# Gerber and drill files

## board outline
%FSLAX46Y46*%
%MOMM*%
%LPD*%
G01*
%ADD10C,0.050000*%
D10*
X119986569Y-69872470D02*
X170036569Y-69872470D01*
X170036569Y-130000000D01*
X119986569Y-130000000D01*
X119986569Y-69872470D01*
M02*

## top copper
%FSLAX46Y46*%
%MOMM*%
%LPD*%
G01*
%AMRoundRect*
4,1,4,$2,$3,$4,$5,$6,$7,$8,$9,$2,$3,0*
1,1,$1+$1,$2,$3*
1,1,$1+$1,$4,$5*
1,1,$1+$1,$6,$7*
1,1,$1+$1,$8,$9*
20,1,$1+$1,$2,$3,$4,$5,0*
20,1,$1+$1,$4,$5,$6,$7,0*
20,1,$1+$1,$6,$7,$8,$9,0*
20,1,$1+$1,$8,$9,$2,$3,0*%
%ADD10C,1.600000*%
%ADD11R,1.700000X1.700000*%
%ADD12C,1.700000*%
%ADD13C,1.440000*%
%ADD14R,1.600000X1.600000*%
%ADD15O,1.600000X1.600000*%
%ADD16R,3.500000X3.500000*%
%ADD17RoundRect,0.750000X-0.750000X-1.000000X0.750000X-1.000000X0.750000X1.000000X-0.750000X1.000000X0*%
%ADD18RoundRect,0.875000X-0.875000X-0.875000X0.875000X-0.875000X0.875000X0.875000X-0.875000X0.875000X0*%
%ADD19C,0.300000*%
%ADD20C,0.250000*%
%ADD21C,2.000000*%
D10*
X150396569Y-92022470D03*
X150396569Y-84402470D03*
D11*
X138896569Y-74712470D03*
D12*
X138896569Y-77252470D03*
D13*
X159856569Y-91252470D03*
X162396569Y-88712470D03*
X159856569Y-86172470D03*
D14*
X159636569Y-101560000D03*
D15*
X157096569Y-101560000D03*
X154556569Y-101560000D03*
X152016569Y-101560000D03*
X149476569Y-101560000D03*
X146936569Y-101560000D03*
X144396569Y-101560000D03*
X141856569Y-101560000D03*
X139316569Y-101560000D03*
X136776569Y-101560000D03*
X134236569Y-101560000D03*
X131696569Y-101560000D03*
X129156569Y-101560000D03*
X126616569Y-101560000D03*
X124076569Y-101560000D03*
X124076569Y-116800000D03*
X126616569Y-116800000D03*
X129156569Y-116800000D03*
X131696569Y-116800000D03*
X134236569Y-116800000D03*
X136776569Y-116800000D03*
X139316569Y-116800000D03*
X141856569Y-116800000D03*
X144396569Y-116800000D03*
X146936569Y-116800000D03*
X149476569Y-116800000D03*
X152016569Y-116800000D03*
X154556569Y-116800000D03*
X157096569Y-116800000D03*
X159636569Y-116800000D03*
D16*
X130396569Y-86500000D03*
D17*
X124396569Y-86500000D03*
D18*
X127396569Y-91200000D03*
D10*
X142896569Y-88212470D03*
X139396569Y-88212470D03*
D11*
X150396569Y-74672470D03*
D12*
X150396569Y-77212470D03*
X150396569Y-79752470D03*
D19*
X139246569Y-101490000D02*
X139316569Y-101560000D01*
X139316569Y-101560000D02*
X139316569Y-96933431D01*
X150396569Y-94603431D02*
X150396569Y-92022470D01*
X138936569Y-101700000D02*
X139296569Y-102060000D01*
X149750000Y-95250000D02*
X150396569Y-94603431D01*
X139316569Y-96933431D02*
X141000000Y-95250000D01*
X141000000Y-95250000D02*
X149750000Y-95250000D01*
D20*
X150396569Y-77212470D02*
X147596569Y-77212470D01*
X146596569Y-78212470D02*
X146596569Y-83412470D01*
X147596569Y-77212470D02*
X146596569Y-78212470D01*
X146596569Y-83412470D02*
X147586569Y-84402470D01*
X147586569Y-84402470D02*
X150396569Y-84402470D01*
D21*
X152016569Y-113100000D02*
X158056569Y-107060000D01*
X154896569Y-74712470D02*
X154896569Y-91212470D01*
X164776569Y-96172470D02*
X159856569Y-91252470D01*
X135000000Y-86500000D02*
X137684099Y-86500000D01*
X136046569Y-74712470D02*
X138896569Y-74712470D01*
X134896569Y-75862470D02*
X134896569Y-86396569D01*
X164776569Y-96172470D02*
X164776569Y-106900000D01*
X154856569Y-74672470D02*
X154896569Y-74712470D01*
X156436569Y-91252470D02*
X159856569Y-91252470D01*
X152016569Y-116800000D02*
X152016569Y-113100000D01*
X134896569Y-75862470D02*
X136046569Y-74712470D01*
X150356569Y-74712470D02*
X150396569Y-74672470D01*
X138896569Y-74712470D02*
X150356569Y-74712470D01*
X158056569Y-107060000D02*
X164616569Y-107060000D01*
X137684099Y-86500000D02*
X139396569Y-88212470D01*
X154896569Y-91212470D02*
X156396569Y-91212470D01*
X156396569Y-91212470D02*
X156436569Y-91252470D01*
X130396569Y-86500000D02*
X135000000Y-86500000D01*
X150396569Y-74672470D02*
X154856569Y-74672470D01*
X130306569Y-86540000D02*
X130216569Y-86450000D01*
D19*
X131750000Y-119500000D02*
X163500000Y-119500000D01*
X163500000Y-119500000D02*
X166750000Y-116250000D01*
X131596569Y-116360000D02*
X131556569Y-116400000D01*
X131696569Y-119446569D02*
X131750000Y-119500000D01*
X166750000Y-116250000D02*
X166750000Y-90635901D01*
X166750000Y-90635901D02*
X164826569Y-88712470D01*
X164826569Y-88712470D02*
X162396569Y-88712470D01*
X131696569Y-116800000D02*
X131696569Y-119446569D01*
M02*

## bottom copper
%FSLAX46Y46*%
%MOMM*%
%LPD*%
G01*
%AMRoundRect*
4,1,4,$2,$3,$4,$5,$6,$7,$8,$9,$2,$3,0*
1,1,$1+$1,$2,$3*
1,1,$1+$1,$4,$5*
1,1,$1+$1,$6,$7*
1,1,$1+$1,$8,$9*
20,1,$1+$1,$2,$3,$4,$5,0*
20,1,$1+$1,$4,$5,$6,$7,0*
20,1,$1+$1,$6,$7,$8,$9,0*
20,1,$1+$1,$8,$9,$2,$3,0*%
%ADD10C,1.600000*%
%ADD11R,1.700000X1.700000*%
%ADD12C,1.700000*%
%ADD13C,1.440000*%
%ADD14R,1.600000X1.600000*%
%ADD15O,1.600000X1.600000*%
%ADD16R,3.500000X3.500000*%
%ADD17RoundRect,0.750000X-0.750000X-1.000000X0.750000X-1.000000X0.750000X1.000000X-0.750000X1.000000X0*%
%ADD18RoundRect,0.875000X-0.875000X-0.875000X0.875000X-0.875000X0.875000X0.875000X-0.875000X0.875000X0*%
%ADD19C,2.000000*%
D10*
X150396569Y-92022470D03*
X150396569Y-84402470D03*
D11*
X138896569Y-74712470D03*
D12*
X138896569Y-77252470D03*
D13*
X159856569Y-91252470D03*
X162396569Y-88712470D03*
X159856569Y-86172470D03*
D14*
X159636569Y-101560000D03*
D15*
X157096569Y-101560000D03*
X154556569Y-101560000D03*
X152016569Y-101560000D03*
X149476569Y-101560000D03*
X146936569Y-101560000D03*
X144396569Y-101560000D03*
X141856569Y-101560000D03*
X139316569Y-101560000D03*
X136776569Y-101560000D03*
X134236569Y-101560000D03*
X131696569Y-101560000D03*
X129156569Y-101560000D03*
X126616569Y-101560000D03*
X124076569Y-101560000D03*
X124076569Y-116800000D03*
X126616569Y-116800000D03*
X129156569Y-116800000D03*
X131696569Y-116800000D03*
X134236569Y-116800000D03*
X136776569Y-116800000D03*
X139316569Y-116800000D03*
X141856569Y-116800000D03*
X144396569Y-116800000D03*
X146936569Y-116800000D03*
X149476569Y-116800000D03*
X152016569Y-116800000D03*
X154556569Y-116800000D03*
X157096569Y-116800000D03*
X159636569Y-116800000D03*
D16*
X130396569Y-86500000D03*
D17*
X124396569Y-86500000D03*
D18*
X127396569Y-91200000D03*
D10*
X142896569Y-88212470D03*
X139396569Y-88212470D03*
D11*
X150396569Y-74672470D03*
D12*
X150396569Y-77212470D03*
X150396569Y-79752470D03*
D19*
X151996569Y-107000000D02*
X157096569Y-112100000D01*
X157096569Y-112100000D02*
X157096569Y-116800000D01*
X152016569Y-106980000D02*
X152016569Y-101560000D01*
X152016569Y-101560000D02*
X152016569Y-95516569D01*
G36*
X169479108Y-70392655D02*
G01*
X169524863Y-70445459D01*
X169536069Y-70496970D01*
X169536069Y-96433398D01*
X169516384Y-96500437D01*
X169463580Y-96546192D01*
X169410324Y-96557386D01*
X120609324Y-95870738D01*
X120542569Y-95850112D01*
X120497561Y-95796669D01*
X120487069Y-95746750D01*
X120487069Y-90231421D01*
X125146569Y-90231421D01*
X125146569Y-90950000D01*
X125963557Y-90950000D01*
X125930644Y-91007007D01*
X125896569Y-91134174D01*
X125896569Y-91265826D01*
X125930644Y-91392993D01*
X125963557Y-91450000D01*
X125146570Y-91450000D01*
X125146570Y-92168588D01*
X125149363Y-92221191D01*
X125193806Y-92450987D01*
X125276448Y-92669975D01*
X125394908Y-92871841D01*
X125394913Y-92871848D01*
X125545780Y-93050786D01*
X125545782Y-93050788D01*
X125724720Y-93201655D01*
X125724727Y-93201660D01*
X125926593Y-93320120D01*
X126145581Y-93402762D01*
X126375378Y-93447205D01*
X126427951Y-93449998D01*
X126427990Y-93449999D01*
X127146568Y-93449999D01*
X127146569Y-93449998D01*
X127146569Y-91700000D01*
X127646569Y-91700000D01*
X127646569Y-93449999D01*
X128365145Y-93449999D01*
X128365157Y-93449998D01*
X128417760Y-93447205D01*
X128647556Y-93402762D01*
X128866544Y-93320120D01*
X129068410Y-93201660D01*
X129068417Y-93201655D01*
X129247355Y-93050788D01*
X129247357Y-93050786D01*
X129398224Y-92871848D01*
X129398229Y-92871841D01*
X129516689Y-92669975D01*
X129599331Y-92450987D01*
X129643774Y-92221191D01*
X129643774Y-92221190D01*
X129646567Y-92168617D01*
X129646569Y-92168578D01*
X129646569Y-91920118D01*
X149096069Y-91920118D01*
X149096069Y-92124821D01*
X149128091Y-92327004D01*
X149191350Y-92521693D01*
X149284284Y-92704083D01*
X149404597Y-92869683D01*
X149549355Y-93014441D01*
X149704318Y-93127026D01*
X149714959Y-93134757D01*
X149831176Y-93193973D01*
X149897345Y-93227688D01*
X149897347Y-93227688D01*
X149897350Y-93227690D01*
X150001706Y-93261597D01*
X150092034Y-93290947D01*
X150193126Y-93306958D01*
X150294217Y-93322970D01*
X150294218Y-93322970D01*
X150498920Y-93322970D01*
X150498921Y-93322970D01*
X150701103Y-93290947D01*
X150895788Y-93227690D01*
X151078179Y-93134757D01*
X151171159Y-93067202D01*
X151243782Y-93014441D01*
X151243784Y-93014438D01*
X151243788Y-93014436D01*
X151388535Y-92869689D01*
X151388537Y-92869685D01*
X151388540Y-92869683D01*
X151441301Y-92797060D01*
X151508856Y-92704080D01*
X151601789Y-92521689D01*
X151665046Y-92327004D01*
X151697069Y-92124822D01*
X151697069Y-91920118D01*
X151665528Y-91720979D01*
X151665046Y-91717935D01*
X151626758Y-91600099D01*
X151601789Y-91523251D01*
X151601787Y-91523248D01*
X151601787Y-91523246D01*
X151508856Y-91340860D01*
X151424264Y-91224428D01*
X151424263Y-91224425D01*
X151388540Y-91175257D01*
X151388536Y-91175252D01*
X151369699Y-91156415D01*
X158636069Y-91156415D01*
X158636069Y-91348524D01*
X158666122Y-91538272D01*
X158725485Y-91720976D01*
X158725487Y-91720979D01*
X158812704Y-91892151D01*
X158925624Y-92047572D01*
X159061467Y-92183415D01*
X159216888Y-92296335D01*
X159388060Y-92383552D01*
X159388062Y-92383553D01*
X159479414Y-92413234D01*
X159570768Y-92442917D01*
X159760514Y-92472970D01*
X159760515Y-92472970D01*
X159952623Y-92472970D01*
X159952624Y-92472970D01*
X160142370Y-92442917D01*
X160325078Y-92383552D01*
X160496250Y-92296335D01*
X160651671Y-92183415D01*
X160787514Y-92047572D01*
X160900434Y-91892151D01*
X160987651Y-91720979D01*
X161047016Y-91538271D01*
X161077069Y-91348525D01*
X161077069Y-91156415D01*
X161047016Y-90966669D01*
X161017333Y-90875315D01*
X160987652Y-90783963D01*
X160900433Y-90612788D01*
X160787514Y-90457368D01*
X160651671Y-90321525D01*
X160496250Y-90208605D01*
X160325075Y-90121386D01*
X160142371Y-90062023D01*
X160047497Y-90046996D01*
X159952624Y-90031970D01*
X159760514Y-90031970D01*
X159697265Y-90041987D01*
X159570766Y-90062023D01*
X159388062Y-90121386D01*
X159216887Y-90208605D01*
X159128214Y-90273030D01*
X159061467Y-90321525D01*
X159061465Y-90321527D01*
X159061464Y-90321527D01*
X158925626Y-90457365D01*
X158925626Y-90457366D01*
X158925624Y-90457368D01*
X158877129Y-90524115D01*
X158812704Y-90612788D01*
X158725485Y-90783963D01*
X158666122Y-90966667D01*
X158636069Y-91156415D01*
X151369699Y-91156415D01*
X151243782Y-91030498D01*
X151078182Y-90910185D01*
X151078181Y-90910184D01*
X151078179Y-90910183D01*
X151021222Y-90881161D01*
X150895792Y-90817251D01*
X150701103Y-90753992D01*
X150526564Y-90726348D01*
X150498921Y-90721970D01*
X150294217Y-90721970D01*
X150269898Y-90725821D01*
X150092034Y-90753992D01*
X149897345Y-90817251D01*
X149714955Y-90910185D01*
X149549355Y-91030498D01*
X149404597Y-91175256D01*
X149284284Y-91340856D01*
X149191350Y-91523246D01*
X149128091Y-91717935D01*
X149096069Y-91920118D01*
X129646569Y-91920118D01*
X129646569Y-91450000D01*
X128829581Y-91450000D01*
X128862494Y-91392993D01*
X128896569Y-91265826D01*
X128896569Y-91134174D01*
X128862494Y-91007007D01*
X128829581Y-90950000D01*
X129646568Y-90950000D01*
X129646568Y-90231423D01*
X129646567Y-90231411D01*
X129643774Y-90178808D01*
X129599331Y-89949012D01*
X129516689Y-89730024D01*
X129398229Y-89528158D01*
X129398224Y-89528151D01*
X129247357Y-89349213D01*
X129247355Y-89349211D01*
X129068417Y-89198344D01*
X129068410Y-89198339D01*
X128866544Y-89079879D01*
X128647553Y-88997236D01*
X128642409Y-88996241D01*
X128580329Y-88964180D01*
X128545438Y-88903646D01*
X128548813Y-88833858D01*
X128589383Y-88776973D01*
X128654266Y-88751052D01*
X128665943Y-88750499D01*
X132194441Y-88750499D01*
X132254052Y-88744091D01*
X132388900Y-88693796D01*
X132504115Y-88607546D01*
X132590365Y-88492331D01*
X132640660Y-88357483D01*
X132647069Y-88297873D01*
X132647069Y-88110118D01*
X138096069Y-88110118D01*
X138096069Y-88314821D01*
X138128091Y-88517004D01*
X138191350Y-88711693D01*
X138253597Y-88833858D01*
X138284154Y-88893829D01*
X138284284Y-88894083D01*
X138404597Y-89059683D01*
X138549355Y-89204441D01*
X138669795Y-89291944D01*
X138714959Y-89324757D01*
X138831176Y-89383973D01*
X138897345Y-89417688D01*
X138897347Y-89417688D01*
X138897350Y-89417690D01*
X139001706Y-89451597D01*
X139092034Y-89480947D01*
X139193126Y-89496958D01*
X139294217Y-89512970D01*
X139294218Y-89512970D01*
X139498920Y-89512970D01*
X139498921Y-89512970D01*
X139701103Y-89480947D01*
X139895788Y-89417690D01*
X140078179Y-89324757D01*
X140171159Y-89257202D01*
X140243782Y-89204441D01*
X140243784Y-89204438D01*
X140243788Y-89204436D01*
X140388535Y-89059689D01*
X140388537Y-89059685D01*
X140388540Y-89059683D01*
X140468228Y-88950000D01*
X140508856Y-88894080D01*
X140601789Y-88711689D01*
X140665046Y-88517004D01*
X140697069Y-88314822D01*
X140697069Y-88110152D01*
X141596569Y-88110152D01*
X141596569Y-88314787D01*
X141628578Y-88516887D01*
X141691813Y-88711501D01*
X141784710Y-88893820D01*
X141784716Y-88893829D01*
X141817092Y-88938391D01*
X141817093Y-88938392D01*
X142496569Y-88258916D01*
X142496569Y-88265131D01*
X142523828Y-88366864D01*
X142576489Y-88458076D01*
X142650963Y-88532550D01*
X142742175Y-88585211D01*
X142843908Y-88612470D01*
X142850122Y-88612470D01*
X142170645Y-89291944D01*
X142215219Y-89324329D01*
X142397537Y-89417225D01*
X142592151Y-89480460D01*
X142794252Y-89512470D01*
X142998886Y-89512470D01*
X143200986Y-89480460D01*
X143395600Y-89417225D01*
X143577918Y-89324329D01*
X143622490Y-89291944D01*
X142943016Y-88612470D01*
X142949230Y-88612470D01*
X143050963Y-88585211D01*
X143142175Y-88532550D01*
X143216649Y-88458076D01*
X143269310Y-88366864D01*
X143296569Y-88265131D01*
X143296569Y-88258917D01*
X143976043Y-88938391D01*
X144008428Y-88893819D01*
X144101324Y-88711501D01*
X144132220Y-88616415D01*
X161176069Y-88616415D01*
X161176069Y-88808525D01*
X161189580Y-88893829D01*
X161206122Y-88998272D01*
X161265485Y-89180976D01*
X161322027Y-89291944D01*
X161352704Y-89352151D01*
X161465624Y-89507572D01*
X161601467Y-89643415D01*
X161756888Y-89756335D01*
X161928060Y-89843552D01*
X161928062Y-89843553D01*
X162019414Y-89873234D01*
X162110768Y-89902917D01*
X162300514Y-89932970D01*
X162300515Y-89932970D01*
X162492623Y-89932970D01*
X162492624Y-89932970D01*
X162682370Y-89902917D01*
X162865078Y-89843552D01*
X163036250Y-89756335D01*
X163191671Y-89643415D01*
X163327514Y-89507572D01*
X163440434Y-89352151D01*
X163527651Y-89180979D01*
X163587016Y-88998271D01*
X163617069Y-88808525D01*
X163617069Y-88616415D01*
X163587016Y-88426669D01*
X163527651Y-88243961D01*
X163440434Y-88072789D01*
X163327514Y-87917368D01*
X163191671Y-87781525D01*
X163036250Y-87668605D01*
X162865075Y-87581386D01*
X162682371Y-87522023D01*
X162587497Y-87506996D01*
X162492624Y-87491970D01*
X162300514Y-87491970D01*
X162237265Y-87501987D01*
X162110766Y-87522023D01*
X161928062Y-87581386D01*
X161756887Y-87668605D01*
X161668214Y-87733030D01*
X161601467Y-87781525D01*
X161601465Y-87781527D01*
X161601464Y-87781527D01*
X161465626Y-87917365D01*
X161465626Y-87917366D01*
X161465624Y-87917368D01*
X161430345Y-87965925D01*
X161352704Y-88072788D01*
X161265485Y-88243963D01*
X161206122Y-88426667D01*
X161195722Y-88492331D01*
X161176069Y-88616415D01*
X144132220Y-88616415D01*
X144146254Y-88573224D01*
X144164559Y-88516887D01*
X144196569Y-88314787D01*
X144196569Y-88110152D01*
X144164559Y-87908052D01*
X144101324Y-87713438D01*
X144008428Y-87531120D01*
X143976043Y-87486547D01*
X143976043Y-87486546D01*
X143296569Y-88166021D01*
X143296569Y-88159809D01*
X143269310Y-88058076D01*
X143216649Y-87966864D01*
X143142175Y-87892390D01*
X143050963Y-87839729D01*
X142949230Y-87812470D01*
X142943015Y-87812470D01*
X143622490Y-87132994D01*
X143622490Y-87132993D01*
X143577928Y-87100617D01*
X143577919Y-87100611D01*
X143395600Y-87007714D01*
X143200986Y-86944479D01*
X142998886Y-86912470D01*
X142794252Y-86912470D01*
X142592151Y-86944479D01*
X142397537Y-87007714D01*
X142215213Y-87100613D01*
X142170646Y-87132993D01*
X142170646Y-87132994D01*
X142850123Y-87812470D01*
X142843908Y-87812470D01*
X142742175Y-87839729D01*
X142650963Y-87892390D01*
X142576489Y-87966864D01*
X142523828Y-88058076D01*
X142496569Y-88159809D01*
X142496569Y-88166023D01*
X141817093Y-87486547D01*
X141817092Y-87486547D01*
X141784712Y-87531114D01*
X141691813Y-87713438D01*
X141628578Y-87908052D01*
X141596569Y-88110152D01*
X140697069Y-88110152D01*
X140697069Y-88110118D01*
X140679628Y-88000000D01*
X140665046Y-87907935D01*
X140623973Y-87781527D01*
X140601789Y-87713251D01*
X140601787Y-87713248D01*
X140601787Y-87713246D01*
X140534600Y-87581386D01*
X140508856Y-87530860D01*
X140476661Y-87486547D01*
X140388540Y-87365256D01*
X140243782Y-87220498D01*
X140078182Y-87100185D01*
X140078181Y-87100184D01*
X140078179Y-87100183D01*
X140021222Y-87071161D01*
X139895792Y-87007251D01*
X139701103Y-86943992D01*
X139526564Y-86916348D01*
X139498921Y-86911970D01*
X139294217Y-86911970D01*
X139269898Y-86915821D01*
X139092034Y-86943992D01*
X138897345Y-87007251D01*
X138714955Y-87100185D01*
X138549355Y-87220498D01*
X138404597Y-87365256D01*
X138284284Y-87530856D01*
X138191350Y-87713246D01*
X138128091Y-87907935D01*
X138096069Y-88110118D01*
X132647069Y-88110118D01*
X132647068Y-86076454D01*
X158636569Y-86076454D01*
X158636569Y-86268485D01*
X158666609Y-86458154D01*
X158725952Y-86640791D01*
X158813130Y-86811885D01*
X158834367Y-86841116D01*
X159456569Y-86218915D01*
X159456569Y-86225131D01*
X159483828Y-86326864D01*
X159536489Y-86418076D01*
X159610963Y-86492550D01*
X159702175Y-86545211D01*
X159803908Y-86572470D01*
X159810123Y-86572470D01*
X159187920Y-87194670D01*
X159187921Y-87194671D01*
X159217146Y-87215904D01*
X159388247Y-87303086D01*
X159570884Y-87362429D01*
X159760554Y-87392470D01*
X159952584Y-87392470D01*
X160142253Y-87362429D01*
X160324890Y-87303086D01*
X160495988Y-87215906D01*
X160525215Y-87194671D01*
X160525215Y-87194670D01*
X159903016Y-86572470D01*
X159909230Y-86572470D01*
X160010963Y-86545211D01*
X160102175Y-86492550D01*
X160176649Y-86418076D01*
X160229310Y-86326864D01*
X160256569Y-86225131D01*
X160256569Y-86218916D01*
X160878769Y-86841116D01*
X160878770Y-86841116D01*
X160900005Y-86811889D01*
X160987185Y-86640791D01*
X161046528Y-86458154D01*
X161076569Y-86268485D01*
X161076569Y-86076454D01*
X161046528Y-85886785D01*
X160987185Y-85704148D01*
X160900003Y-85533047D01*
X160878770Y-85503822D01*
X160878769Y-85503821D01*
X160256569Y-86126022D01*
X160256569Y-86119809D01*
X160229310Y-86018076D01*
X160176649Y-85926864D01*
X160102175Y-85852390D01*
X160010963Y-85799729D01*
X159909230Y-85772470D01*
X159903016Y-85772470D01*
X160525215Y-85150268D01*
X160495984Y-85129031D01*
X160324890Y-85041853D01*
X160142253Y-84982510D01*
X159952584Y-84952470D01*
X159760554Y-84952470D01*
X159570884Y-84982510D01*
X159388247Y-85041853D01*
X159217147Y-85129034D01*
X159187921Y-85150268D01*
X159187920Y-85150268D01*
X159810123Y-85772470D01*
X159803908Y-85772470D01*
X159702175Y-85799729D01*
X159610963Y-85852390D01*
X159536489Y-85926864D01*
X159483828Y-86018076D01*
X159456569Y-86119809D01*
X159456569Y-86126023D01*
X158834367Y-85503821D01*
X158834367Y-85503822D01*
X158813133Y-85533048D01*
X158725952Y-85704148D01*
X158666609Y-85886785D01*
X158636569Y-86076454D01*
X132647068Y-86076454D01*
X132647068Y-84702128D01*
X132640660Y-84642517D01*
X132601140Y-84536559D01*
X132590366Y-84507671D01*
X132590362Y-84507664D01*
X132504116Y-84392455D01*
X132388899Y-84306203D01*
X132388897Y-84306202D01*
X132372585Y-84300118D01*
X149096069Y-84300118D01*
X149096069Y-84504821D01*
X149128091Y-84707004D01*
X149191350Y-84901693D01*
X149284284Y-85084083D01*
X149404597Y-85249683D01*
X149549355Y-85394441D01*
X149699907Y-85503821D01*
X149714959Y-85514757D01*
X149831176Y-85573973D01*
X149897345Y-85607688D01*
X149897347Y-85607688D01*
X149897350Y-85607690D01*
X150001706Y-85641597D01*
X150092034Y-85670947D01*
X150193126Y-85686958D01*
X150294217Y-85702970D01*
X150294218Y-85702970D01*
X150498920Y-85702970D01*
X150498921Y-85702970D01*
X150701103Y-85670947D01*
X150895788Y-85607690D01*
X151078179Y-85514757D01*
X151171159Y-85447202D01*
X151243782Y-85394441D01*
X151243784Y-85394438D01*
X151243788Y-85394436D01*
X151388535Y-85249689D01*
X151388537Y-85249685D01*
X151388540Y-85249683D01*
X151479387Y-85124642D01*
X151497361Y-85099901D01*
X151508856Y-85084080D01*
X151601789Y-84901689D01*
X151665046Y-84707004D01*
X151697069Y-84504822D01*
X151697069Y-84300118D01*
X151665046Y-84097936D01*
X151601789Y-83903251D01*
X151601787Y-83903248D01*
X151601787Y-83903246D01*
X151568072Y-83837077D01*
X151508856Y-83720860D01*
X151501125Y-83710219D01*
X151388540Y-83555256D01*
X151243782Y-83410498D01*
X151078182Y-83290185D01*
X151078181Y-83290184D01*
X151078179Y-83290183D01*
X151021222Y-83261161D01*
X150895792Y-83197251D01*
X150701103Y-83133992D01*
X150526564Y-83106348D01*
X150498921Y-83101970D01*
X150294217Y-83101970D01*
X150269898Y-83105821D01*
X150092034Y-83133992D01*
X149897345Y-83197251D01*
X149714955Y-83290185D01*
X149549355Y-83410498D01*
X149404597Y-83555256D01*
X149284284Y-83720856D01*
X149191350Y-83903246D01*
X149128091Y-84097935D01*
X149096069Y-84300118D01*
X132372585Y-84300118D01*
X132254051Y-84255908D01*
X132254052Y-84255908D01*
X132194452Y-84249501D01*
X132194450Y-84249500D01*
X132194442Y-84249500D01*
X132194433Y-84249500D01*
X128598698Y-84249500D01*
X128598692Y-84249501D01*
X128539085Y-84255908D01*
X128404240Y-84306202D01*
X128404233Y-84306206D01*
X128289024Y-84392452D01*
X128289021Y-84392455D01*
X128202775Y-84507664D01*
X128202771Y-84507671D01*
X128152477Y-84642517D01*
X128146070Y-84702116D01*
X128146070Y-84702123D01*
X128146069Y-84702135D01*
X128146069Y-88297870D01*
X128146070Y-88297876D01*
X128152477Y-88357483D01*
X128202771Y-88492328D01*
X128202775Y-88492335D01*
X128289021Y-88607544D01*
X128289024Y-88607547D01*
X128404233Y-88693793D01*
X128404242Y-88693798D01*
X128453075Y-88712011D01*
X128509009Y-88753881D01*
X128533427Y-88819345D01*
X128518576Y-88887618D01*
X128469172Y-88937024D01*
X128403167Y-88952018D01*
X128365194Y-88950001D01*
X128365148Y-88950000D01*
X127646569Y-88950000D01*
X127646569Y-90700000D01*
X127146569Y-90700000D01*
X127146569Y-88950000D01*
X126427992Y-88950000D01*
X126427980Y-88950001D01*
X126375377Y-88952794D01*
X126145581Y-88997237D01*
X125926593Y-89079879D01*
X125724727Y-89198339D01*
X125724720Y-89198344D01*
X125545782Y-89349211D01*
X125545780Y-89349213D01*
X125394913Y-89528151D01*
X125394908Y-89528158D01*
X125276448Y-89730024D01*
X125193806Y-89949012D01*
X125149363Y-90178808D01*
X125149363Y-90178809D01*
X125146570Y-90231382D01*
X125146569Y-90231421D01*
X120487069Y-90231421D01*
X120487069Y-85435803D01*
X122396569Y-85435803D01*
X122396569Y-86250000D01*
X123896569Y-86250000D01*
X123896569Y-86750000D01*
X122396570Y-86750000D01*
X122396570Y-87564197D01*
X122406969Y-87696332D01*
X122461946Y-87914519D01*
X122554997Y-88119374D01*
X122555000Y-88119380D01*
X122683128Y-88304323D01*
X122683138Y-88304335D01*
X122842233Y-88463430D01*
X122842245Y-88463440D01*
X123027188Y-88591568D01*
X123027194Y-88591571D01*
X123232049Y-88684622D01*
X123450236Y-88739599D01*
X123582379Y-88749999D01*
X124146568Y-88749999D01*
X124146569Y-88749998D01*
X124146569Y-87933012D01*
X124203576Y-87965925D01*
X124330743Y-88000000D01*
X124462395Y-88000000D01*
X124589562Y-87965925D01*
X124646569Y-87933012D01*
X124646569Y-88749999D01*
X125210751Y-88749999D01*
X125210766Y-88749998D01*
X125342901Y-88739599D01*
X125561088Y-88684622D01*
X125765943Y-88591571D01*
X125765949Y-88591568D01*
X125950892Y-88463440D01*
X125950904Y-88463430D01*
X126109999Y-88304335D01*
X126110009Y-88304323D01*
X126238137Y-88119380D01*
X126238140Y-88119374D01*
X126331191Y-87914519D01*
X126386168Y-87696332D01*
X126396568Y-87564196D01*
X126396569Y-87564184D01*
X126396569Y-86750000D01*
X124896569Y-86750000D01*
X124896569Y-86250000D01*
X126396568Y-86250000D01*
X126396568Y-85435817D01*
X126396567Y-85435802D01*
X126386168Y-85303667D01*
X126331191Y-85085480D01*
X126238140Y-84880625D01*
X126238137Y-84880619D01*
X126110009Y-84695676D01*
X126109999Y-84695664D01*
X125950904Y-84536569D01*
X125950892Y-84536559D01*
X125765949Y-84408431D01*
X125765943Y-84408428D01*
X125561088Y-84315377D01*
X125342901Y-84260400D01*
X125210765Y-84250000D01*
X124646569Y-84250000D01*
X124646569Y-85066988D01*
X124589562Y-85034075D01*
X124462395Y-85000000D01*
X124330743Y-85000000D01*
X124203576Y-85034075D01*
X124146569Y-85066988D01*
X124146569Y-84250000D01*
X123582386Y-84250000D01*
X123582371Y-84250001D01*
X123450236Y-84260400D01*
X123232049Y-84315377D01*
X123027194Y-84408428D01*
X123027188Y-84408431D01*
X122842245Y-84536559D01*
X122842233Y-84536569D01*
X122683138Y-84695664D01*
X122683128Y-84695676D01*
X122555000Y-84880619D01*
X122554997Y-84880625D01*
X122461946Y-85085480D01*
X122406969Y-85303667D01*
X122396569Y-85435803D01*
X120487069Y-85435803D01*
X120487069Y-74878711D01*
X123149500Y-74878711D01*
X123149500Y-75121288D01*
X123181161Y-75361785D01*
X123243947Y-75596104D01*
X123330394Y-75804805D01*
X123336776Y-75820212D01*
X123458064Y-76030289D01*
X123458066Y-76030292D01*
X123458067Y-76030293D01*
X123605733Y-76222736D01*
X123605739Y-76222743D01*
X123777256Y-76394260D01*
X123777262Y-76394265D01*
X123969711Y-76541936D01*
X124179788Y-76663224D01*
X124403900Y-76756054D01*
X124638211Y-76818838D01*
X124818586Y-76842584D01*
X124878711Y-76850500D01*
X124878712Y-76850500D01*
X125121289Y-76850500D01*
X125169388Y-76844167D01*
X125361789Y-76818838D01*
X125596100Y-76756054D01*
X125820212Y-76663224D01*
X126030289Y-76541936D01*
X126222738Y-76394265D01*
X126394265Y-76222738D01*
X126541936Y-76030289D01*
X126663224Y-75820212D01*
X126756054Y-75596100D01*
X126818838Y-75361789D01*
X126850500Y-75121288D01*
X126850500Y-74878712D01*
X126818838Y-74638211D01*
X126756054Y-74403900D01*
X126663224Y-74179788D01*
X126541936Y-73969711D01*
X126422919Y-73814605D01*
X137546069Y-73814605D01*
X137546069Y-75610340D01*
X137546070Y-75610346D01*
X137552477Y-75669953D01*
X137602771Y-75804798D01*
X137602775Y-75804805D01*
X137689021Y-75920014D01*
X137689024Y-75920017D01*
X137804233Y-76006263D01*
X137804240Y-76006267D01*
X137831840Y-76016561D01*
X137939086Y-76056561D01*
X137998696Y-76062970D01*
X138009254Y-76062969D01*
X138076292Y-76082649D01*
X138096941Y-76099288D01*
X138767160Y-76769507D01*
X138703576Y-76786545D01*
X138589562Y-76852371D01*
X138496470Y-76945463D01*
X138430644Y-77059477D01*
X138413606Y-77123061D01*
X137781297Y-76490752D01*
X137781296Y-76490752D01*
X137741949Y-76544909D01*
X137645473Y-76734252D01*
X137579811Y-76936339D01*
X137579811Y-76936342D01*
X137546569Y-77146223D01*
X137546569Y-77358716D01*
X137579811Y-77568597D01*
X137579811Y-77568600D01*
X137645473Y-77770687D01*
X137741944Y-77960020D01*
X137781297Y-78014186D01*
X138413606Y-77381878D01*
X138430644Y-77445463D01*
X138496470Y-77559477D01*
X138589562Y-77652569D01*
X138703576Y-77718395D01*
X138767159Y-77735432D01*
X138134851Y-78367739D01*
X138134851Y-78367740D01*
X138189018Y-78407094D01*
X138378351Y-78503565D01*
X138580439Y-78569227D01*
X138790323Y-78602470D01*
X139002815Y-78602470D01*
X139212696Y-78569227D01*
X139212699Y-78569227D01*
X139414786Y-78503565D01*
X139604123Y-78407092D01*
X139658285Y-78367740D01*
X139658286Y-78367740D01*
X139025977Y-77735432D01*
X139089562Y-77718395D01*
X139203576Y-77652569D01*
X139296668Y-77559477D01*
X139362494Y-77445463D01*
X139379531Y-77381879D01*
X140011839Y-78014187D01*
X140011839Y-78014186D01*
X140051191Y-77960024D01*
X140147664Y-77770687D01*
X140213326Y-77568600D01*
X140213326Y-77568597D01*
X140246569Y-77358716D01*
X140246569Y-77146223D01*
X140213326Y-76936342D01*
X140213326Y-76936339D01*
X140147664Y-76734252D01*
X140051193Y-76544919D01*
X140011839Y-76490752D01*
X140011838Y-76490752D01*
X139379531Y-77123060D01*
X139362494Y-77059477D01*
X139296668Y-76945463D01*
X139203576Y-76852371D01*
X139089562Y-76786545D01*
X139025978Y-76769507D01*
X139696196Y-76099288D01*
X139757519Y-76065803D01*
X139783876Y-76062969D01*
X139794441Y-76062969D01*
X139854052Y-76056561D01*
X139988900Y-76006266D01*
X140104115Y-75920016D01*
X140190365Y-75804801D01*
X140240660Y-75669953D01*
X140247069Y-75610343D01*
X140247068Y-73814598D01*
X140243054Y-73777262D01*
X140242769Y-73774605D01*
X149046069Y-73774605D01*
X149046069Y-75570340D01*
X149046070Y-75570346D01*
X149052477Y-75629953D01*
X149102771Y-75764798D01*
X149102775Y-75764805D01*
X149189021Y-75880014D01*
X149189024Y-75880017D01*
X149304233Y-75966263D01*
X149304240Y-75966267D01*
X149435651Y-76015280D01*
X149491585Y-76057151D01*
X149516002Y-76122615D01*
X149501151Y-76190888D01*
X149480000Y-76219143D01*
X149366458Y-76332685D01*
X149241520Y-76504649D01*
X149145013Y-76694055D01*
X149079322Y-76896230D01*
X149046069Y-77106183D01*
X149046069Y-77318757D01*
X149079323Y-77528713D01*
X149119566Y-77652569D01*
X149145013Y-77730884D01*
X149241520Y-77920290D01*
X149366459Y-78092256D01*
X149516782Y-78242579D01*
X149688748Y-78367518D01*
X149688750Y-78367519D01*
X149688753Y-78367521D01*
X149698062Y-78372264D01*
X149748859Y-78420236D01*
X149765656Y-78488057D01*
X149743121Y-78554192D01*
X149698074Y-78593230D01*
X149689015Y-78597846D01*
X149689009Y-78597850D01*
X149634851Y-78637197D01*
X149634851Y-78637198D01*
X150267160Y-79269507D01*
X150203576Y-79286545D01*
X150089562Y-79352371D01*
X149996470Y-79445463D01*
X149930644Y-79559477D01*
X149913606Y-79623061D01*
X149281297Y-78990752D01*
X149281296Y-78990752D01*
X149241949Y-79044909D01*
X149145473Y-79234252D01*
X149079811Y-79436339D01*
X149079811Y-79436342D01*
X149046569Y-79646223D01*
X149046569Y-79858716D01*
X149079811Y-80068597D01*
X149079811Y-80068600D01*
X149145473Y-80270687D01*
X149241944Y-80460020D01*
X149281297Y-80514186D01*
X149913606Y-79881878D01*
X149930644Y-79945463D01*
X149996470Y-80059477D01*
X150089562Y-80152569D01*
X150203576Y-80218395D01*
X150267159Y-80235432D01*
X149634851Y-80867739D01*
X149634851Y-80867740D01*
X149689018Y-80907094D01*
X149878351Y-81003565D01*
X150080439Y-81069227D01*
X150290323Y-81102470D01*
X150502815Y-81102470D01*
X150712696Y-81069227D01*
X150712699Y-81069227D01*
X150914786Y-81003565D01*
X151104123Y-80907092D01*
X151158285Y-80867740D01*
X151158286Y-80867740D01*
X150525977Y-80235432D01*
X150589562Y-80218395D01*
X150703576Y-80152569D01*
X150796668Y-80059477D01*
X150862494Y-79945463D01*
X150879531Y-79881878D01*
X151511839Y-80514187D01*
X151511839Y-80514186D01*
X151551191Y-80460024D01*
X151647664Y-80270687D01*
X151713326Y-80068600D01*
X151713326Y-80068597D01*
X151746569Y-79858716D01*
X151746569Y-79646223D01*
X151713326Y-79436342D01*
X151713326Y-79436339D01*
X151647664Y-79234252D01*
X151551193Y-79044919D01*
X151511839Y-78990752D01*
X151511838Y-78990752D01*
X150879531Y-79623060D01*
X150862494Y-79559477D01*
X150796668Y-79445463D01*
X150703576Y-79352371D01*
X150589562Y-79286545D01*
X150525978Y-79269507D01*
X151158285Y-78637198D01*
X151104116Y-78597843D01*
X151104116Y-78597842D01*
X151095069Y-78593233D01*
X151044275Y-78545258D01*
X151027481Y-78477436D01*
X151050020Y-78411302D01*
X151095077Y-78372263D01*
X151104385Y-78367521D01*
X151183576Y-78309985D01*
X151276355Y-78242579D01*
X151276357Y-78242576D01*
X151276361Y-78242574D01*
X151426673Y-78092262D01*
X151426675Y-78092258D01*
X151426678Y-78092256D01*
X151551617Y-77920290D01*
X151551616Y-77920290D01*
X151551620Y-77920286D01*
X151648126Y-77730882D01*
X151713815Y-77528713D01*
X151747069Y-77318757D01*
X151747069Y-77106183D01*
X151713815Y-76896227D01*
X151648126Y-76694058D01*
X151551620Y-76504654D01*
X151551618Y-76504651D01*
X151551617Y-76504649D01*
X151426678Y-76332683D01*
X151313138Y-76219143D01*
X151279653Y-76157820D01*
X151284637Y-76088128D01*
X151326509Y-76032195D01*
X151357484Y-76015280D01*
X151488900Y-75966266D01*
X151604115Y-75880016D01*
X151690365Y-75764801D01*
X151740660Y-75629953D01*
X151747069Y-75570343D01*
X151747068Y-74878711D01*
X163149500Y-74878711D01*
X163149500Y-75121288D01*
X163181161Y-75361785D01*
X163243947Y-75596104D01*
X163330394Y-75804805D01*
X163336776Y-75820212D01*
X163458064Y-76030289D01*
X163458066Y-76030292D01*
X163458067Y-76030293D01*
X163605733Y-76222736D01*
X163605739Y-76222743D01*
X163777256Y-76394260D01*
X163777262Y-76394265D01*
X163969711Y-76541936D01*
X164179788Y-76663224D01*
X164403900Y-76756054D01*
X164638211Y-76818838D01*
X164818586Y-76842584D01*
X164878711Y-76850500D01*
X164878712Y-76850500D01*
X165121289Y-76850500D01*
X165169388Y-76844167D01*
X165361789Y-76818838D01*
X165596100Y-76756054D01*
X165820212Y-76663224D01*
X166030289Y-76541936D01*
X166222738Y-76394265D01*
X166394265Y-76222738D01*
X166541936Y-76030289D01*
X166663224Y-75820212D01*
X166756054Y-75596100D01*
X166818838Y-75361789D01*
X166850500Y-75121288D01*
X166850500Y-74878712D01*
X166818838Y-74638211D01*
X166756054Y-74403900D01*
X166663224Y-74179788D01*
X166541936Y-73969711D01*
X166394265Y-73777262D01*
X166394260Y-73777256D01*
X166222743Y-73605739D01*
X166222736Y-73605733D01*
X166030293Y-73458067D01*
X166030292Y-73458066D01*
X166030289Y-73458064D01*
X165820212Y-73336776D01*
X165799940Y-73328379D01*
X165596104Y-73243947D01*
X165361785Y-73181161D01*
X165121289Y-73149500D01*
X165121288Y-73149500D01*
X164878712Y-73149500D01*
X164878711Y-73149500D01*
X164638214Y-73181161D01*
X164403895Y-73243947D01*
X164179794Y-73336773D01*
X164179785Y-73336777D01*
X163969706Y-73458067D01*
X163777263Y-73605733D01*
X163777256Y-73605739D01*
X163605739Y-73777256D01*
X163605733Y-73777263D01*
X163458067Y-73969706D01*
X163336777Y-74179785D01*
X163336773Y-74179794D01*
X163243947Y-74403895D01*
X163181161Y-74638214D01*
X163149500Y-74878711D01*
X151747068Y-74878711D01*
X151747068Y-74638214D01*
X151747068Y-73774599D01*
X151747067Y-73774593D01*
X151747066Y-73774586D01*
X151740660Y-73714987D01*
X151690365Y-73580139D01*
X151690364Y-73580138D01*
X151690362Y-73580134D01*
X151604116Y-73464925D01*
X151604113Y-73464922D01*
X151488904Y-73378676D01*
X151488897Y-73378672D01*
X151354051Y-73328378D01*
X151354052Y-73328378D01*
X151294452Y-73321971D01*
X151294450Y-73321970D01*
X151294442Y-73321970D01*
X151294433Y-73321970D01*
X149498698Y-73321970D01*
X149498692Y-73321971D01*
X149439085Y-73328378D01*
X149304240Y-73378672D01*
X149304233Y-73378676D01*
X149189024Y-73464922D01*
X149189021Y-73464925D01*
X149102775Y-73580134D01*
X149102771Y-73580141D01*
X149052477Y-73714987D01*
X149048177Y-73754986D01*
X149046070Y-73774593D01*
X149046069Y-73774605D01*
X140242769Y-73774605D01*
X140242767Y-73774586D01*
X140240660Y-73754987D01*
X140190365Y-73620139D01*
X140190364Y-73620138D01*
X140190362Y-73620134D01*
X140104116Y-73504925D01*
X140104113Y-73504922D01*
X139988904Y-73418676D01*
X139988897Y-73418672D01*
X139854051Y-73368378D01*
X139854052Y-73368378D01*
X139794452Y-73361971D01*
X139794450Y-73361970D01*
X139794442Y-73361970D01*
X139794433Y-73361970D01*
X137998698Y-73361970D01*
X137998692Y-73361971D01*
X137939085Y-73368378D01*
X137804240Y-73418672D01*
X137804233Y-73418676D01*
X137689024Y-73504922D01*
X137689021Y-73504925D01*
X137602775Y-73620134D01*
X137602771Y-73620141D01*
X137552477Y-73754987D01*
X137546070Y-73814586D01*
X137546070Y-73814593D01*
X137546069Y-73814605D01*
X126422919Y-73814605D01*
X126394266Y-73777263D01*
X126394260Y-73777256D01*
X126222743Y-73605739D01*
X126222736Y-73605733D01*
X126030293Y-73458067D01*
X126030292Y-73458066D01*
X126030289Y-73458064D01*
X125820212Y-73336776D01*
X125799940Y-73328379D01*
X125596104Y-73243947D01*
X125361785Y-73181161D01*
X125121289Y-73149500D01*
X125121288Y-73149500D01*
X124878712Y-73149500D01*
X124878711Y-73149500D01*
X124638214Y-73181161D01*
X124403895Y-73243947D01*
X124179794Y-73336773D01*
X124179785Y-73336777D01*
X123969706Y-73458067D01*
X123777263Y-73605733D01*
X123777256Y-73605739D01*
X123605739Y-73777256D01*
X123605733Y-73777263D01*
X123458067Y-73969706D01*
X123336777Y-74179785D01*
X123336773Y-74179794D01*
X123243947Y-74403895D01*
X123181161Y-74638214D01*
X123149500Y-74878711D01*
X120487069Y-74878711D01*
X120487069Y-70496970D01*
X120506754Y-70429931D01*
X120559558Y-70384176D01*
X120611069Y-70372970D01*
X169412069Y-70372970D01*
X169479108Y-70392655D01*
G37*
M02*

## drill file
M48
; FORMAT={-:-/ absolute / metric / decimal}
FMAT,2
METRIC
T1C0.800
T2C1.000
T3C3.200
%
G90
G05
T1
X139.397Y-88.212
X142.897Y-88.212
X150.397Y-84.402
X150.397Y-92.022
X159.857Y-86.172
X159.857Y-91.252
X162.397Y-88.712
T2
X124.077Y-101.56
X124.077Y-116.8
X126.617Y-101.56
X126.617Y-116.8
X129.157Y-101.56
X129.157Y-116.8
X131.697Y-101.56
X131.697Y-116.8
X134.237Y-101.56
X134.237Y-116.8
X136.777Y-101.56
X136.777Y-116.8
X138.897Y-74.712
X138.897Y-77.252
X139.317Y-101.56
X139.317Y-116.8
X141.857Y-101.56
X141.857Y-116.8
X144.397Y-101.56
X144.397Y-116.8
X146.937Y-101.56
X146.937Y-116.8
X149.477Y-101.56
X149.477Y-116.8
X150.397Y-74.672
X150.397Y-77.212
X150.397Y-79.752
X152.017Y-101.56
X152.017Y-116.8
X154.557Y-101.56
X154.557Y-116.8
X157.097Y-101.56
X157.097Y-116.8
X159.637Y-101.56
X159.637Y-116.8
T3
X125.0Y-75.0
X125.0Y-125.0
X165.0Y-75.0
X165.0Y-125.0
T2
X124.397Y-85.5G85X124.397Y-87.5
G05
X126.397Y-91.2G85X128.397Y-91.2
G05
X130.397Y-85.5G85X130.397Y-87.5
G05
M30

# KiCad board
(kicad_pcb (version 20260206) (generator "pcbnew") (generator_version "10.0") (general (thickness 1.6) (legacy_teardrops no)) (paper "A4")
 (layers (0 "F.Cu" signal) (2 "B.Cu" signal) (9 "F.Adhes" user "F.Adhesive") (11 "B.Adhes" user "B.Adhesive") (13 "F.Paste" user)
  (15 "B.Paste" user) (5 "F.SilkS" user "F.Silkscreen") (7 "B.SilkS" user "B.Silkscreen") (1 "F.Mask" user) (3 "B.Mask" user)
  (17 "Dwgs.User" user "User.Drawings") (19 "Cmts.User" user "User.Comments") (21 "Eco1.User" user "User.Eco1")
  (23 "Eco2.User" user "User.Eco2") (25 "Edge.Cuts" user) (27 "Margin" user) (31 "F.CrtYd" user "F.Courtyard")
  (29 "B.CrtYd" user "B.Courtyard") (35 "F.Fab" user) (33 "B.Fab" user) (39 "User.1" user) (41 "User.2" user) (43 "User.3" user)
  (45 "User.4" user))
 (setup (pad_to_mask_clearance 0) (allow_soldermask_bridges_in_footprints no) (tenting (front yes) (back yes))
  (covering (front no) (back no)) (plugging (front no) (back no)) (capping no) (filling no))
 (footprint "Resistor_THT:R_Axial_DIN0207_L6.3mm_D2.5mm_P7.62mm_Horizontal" (layer "F.Cu") (at 150.396569 92.02247 90)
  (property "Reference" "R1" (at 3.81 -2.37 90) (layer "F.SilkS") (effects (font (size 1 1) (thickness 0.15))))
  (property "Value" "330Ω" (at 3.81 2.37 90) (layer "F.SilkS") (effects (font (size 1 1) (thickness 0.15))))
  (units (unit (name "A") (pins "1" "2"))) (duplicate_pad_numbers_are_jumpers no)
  (pad "1" thru_hole circle (at 0 0 90) (size 1.6 1.6) (drill 0.8) (layers "*.Cu" "*.Mask") (remove_unused_layers no) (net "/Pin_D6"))
  (pad "2" thru_hole circle (at 7.62 0 90) (size 1.6 1.6) (drill 0.8) (layers "*.Cu" "*.Mask") (remove_unused_layers no) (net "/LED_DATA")))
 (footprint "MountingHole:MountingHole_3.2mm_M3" (layer "F.Cu") (at 165 125)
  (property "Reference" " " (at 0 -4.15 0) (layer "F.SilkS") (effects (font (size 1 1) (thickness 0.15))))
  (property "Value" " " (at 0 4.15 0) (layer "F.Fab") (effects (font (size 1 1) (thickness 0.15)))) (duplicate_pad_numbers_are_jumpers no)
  (pad "" np_thru_hole circle (at 0 0) (size 3.2 3.2) (drill 3.2) (layers "*.Cu" "*.Mask")))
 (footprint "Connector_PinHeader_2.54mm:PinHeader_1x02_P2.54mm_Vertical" (layer "F.Cu") (at 138.896569 74.71247)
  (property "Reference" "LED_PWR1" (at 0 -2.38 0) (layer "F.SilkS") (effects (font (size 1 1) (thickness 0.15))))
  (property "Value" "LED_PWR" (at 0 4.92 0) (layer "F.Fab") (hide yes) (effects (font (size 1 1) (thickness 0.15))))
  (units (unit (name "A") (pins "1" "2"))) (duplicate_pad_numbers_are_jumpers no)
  (pad "1" thru_hole rect (at 0 0) (size 1.7 1.7) (drill 1) (layers "*.Cu" "*.Mask") (remove_unused_layers no) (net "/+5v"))
  (pad "2" thru_hole circle (at 0 2.54) (size 1.7 1.7) (drill 1) (layers "*.Cu" "*.Mask") (remove_unused_layers no) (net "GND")))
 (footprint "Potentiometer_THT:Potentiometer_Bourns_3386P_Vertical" (layer "F.Cu") (at 159.856569 91.25247)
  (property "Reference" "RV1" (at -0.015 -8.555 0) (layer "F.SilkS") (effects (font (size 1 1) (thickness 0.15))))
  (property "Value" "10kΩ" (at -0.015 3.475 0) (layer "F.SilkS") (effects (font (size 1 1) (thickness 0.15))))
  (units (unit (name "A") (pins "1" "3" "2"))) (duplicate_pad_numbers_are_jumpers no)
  (pad "1" thru_hole circle (at 0 0) (size 1.44 1.44) (drill 0.8) (layers "*.Cu" "*.Mask") (remove_unused_layers no) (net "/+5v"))
  (pad "2" thru_hole circle (at 2.54 -2.54) (size 1.44 1.44) (drill 0.8) (layers "*.Cu" "*.Mask") (remove_unused_layers no)
   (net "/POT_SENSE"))
  (pad "3" thru_hole circle (at 0 -5.08) (size 1.44 1.44) (drill 0.8) (layers "*.Cu" "*.Mask") (remove_unused_layers no) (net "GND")))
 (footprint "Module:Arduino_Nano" (layer "F.Cu") (at 159.636569 101.56 -90)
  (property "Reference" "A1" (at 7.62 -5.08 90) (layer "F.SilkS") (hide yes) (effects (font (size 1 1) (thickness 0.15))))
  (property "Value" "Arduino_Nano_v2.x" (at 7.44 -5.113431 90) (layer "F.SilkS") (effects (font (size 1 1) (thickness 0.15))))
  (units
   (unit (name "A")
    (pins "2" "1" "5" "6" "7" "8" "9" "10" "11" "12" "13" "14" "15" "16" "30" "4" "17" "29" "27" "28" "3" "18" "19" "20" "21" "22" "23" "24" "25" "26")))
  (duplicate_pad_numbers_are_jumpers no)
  (pad "1" thru_hole rect (at 0 0 270) (size 1.6 1.6) (drill 1) (layers "*.Cu" "*.Mask") (remove_unused_layers no)
   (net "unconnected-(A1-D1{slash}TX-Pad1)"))
  (pad "2" thru_hole oval (at 0 2.54 270) (size 1.6 1.6) (drill 1) (layers "*.Cu" "*.Mask") (remove_unused_layers no)
   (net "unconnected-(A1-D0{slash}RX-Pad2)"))
  (pad "3" thru_hole oval (at 0 5.08 270) (size 1.6 1.6) (drill 1) (layers "*.Cu" "*.Mask") (remove_unused_layers no)
   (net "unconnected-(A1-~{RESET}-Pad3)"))
  (pad "4" thru_hole oval (at 0 7.62 270) (size 1.6 1.6) (drill 1) (layers "*.Cu" "*.Mask") (remove_unused_layers no) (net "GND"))
  (pad "5" thru_hole oval (at 0 10.16 270) (size 1.6 1.6) (drill 1) (layers "*.Cu" "*.Mask") (remove_unused_layers no)
   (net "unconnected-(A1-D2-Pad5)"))
  (pad "6" thru_hole oval (at 0 12.7 270) (size 1.6 1.6) (drill 1) (layers "*.Cu" "*.Mask") (remove_unused_layers no)
   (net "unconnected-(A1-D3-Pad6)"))
  (pad "7" thru_hole oval (at 0 15.24 270) (size 1.6 1.6) (drill 1) (layers "*.Cu" "*.Mask") (remove_unused_layers no)
   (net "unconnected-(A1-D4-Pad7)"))
  (pad "8" thru_hole oval (at 0 17.78 270) (size 1.6 1.6) (drill 1) (layers "*.Cu" "*.Mask") (remove_unused_layers no)
   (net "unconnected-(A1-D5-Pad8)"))
  (pad "9" thru_hole oval (at 0 20.32 270) (size 1.6 1.6) (drill 1) (layers "*.Cu" "*.Mask") (remove_unused_layers no) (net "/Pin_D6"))
  (pad "10" thru_hole oval (at 0 22.86 270) (size 1.6 1.6) (drill 1) (layers "*.Cu" "*.Mask") (remove_unused_layers no)
   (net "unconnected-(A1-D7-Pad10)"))
  (pad "11" thru_hole oval (at 0 25.4 270) (size 1.6 1.6) (drill 1) (layers "*.Cu" "*.Mask") (remove_unused_layers no)
   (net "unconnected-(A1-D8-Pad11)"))
  (pad "12" thru_hole oval (at 0 27.94 270) (size 1.6 1.6) (drill 1) (layers "*.Cu" "*.Mask") (remove_unused_layers no)
   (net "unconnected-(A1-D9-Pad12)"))
  (pad "13" thru_hole oval (at 0 30.48 270) (size 1.6 1.6) (drill 1) (layers "*.Cu" "*.Mask") (remove_unused_layers no)
   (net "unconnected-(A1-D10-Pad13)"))
  (pad "14" thru_hole oval (at 0 33.02 270) (size 1.6 1.6) (drill 1) (layers "*.Cu" "*.Mask") (remove_unused_layers no)
   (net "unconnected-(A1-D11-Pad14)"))
  (pad "15" thru_hole oval (at 0 35.56 270) (size 1.6 1.6) (drill 1) (layers "*.Cu" "*.Mask") (remove_unused_layers no)
   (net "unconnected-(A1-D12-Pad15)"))
  (pad "16" thru_hole oval (at 15.24 35.56 270) (size 1.6 1.6) (drill 1) (layers "*.Cu" "*.Mask") (remove_unused_layers no)
   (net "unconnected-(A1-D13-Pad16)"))
  (pad "17" thru_hole oval (at 15.24 33.02 270) (size 1.6 1.6) (drill 1) (layers "*.Cu" "*.Mask") (remove_unused_layers no)
   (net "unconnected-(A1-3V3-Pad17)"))
  (pad "18" thru_hole oval (at 15.24 30.48 270) (size 1.6 1.6) (drill 1) (layers "*.Cu" "*.Mask") (remove_unused_layers no)
   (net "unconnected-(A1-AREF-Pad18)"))
  (pad "19" thru_hole oval (at 15.24 27.94 270) (size 1.6 1.6) (drill 1) (layers "*.Cu" "*.Mask") (remove_unused_layers no)
   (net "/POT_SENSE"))
  (pad "20" thru_hole oval (at 15.24 25.4 270) (size 1.6 1.6) (drill 1) (layers "*.Cu" "*.Mask") (remove_unused_layers no)
   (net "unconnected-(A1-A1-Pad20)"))
  (pad "21" thru_hole oval (at 15.24 22.86 270) (size 1.6 1.6) (drill 1) (layers "*.Cu" "*.Mask") (remove_unused_layers no)
   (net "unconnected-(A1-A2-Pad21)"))
  (pad "22" thru_hole oval (at 15.24 20.32 270) (size 1.6 1.6) (drill 1) (layers "*.Cu" "*.Mask") (remove_unused_layers no)
   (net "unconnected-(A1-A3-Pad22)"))
  (pad "23" thru_hole oval (at 15.24 17.78 270) (size 1.6 1.6) (drill 1) (layers "*.Cu" "*.Mask") (remove_unused_layers no)
   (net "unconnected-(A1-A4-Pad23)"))
  (pad "24" thru_hole oval (at 15.24 15.24 270) (size 1.6 1.6) (drill 1) (layers "*.Cu" "*.Mask") (remove_unused_layers no)
   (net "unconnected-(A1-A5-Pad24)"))
  (pad "25" thru_hole oval (at 15.24 12.7 270) (size 1.6 1.6) (drill 1) (layers "*.Cu" "*.Mask") (remove_unused_layers no)
   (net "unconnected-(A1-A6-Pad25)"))
  (pad "26" thru_hole oval (at 15.24 10.16 270) (size 1.6 1.6) (drill 1) (layers "*.Cu" "*.Mask") (remove_unused_layers no)
   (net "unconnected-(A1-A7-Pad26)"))
  (pad "27" thru_hole oval (at 15.24 7.62 270) (size 1.6 1.6) (drill 1) (layers "*.Cu" "*.Mask") (remove_unused_layers no) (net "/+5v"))
  (pad "28" thru_hole oval (at 15.24 5.08 270) (size 1.6 1.6) (drill 1) (layers "*.Cu" "*.Mask") (remove_unused_layers no)
   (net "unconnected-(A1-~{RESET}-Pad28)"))
  (pad "29" thru_hole oval (at 15.24 2.54 270) (size 1.6 1.6) (drill 1) (layers "*.Cu" "*.Mask") (remove_unused_layers no) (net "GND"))
  (pad "30" thru_hole oval (at 15.24 0 270) (size 1.6 1.6) (drill 1) (layers "*.Cu" "*.Mask") (remove_unused_layers no)
   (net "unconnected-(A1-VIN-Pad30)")))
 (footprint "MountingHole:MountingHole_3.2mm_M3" (layer "F.Cu") (at 125 75)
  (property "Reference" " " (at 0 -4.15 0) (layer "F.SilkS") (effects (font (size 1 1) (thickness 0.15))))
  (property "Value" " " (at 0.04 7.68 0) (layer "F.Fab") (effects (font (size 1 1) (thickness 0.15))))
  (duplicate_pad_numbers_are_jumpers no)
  (pad "" np_thru_hole circle (at 0 0) (size 3.2 3.2) (drill 3.2) (layers "*.Cu" "*.Mask")))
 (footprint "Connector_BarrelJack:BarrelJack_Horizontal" (layer "F.Cu") (at 130.396569 86.5)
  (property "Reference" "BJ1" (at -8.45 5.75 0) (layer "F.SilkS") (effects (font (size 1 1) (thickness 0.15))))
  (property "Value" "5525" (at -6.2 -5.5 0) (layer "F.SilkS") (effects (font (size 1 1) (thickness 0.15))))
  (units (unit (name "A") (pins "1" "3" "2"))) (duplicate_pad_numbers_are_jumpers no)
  (pad "1" thru_hole rect (at 0 0) (size 3.5 3.5) (drill oval 1 3) (layers "*.Cu" "*.Mask") (remove_unused_layers no) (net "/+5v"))
  (pad "2" thru_hole roundrect (at -6 0) (size 3 3.5) (drill oval 1 3) (layers "*.Cu" "*.Mask") (remove_unused_layers no)
   (roundrect_rratio 0.25) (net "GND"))
  (pad "3" thru_hole roundrect (at -3 4.7) (size 3.5 3.5) (drill oval 3 1) (layers "*.Cu" "*.Mask") (remove_unused_layers no)
   (roundrect_rratio 0.25) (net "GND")))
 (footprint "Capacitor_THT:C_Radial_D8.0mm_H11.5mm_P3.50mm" (layer "F.Cu") (at 142.896569 88.21247 180)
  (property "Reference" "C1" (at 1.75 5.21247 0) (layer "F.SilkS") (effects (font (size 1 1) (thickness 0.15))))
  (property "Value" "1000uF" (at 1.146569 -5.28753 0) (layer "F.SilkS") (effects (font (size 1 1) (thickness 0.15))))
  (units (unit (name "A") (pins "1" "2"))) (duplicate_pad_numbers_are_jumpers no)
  (pad "1" thru_hole circle (at 0 0 180) (size 1.6 1.6) (drill 0.8) (layers "*.Cu" "*.Mask") (remove_unused_layers no) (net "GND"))
  (pad "2" thru_hole circle (at 3.5 0 180) (size 1.6 1.6) (drill 0.8) (layers "*.Cu" "*.Mask") (remove_unused_layers no) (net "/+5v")))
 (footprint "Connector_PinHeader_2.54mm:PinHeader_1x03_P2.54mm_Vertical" (layer "F.Cu") (at 150.396569 74.67247)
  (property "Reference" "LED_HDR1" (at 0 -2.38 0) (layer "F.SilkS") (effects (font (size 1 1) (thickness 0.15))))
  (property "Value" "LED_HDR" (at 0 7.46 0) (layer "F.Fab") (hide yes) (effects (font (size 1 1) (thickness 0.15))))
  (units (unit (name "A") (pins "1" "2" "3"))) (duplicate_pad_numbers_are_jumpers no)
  (pad "1" thru_hole rect (at 0 0) (size 1.7 1.7) (drill 1) (layers "*.Cu" "*.Mask") (remove_unused_layers no) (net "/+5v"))
  (pad "2" thru_hole circle (at 0 2.54) (size 1.7 1.7) (drill 1) (layers "*.Cu" "*.Mask") (remove_unused_layers no) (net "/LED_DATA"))
  (pad "3" thru_hole circle (at 0 5.08) (size 1.7 1.7) (drill 1) (layers "*.Cu" "*.Mask") (remove_unused_layers no) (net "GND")))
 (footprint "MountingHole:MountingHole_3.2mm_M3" (layer "F.Cu") (at 165 75)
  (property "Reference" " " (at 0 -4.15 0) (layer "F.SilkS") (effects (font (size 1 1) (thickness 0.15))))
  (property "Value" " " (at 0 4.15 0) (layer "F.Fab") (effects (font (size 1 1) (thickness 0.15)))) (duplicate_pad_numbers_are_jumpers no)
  (pad "" np_thru_hole circle (at 0 0) (size 3.2 3.2) (drill 3.2) (layers "*.Cu" "*.Mask")))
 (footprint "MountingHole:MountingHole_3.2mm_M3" (layer "F.Cu") (at 125 125)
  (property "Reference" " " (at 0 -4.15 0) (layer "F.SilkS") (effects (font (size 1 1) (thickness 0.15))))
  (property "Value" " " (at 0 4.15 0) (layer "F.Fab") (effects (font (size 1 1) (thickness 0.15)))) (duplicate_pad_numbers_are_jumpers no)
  (pad "" np_thru_hole circle (at 0 0) (size 3.2 3.2) (drill 3.2) (layers "*.Cu" "*.Mask")))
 (gr_rect (start 119.986569 69.87247) (end 170.036569 130) (stroke (width 0.05) (type default)) (fill no) (layer "Edge.Cuts"))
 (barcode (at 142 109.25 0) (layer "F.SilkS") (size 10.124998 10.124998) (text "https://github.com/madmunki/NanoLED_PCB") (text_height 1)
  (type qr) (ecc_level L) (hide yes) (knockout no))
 (segment (start 139.246569 101.49) (end 139.316569 101.56) (width 0.3) (layer "F.Cu") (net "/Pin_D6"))
 (segment (start 139.316569 101.56) (end 139.316569 96.933431) (width 0.3) (layer "F.Cu") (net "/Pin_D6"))
 (segment (start 150.396569 94.603431) (end 150.396569 92.02247) (width 0.3) (layer "F.Cu") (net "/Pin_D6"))
 (segment (start 138.936569 101.7) (end 139.296569 102.06) (width 0.3) (layer "F.Cu") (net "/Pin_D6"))
 (segment (start 149.75 95.25) (end 150.396569 94.603431) (width 0.3) (layer "F.Cu") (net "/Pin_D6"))
 (segment (start 139.316569 96.933431) (end 141 95.25) (width 0.3) (layer "F.Cu") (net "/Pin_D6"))
 (segment (start 141 95.25) (end 149.75 95.25) (width 0.3) (layer "F.Cu") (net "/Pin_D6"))
 (segment (start 150.396569 77.21247) (end 147.596569 77.21247) (width 0.25) (layer "F.Cu") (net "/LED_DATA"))
 (segment (start 146.596569 78.21247) (end 146.596569 83.41247) (width 0.25) (layer "F.Cu") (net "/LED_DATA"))
 (segment (start 147.596569 77.21247) (end 146.596569 78.21247) (width 0.25) (layer "F.Cu") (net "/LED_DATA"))
 (segment (start 146.596569 83.41247) (end 147.586569 84.40247) (width 0.25) (layer "F.Cu") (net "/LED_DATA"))
 (segment (start 147.586569 84.40247) (end 150.396569 84.40247) (width 0.25) (layer "F.Cu") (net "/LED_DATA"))
 (segment (start 152.016569 113.1) (end 158.056569 107.06) (width 2) (layer "F.Cu") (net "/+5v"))
 (segment (start 154.896569 74.71247) (end 154.896569 91.21247) (width 2) (layer "F.Cu") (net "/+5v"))
 (segment (start 164.776569 96.17247) (end 159.856569 91.25247) (width 2) (layer "F.Cu") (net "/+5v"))
 (segment (start 135 86.5) (end 137.684099 86.5) (width 2) (layer "F.Cu") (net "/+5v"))
 (segment (start 136.046569 74.71247) (end 138.896569 74.71247) (width 2) (layer "F.Cu") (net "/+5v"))
 (segment (start 134.896569 75.86247) (end 134.896569 86.396569) (width 2) (layer "F.Cu") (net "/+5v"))
 (segment (start 164.776569 96.17247) (end 164.776569 106.9) (width 2) (layer "F.Cu") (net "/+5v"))
 (segment (start 154.856569 74.67247) (end 154.896569 74.71247) (width 2) (layer "F.Cu") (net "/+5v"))
 (segment (start 156.436569 91.25247) (end 159.856569 91.25247) (width 2) (layer "F.Cu") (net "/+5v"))
 (segment (start 152.016569 116.8) (end 152.016569 113.1) (width 2) (layer "F.Cu") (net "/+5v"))
 (segment (start 134.896569 75.86247) (end 136.046569 74.71247) (width 2) (layer "F.Cu") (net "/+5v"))
 (segment (start 150.356569 74.71247) (end 150.396569 74.67247) (width 2) (layer "F.Cu") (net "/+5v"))
 (segment (start 138.896569 74.71247) (end 150.356569 74.71247) (width 2) (layer "F.Cu") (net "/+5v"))
 (segment (start 158.056569 107.06) (end 164.616569 107.06) (width 2) (layer "F.Cu") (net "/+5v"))
 (segment (start 137.684099 86.5) (end 139.396569 88.21247) (width 2) (layer "F.Cu") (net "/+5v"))
 (segment (start 154.896569 91.21247) (end 156.396569 91.21247) (width 2) (layer "F.Cu") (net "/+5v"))
 (segment (start 156.396569 91.21247) (end 156.436569 91.25247) (width 2) (layer "F.Cu") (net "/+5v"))
 (segment (start 130.396569 86.5) (end 135 86.5) (width 2) (layer "F.Cu") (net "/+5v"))
 (segment (start 150.396569 74.67247) (end 154.856569 74.67247) (width 2) (layer "F.Cu") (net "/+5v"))
 (segment (start 130.306569 86.54) (end 130.216569 86.45) (width 2) (layer "F.Cu") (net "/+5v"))
 (segment (start 151.996569 107) (end 157.096569 112.1) (width 2) (layer "B.Cu") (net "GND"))
 (segment (start 157.096569 112.1) (end 157.096569 116.8) (width 2) (layer "B.Cu") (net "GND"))
 (segment (start 152.016569 106.98) (end 152.016569 101.56) (width 2) (layer "B.Cu") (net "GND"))
 (segment (start 152.016569 101.56) (end 152.016569 95.516569) (width 2) (layer "B.Cu") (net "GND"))
 (segment (start 131.75 119.5) (end 163.5 119.5) (width 0.3) (layer "F.Cu") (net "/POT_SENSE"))
 (segment (start 163.5 119.5) (end 166.75 116.25) (width 0.3) (layer "F.Cu") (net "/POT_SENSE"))
 (segment (start 131.596569 116.36) (end 131.556569 116.4) (width 0.3) (layer "F.Cu") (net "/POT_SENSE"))
 (segment (start 131.696569 119.446569) (end 131.75 119.5) (width 0.3) (layer "F.Cu") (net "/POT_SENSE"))
 (segment (start 166.75 116.25) (end 166.75 90.635901) (width 0.3) (layer "F.Cu") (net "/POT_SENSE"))
 (segment (start 166.75 90.635901) (end 164.826569 88.71247) (width 0.3) (layer "F.Cu") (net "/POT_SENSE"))
 (segment (start 164.826569 88.71247) (end 162.396569 88.71247) (width 0.3) (layer "F.Cu") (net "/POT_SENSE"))
 (segment (start 131.696569 116.8) (end 131.696569 119.446569) (width 0.3) (layer "F.Cu") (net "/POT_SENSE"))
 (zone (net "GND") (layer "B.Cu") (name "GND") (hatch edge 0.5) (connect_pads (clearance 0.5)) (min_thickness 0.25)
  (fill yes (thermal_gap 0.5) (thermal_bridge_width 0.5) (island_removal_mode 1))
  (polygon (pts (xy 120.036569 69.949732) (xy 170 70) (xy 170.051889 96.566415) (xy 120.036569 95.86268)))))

